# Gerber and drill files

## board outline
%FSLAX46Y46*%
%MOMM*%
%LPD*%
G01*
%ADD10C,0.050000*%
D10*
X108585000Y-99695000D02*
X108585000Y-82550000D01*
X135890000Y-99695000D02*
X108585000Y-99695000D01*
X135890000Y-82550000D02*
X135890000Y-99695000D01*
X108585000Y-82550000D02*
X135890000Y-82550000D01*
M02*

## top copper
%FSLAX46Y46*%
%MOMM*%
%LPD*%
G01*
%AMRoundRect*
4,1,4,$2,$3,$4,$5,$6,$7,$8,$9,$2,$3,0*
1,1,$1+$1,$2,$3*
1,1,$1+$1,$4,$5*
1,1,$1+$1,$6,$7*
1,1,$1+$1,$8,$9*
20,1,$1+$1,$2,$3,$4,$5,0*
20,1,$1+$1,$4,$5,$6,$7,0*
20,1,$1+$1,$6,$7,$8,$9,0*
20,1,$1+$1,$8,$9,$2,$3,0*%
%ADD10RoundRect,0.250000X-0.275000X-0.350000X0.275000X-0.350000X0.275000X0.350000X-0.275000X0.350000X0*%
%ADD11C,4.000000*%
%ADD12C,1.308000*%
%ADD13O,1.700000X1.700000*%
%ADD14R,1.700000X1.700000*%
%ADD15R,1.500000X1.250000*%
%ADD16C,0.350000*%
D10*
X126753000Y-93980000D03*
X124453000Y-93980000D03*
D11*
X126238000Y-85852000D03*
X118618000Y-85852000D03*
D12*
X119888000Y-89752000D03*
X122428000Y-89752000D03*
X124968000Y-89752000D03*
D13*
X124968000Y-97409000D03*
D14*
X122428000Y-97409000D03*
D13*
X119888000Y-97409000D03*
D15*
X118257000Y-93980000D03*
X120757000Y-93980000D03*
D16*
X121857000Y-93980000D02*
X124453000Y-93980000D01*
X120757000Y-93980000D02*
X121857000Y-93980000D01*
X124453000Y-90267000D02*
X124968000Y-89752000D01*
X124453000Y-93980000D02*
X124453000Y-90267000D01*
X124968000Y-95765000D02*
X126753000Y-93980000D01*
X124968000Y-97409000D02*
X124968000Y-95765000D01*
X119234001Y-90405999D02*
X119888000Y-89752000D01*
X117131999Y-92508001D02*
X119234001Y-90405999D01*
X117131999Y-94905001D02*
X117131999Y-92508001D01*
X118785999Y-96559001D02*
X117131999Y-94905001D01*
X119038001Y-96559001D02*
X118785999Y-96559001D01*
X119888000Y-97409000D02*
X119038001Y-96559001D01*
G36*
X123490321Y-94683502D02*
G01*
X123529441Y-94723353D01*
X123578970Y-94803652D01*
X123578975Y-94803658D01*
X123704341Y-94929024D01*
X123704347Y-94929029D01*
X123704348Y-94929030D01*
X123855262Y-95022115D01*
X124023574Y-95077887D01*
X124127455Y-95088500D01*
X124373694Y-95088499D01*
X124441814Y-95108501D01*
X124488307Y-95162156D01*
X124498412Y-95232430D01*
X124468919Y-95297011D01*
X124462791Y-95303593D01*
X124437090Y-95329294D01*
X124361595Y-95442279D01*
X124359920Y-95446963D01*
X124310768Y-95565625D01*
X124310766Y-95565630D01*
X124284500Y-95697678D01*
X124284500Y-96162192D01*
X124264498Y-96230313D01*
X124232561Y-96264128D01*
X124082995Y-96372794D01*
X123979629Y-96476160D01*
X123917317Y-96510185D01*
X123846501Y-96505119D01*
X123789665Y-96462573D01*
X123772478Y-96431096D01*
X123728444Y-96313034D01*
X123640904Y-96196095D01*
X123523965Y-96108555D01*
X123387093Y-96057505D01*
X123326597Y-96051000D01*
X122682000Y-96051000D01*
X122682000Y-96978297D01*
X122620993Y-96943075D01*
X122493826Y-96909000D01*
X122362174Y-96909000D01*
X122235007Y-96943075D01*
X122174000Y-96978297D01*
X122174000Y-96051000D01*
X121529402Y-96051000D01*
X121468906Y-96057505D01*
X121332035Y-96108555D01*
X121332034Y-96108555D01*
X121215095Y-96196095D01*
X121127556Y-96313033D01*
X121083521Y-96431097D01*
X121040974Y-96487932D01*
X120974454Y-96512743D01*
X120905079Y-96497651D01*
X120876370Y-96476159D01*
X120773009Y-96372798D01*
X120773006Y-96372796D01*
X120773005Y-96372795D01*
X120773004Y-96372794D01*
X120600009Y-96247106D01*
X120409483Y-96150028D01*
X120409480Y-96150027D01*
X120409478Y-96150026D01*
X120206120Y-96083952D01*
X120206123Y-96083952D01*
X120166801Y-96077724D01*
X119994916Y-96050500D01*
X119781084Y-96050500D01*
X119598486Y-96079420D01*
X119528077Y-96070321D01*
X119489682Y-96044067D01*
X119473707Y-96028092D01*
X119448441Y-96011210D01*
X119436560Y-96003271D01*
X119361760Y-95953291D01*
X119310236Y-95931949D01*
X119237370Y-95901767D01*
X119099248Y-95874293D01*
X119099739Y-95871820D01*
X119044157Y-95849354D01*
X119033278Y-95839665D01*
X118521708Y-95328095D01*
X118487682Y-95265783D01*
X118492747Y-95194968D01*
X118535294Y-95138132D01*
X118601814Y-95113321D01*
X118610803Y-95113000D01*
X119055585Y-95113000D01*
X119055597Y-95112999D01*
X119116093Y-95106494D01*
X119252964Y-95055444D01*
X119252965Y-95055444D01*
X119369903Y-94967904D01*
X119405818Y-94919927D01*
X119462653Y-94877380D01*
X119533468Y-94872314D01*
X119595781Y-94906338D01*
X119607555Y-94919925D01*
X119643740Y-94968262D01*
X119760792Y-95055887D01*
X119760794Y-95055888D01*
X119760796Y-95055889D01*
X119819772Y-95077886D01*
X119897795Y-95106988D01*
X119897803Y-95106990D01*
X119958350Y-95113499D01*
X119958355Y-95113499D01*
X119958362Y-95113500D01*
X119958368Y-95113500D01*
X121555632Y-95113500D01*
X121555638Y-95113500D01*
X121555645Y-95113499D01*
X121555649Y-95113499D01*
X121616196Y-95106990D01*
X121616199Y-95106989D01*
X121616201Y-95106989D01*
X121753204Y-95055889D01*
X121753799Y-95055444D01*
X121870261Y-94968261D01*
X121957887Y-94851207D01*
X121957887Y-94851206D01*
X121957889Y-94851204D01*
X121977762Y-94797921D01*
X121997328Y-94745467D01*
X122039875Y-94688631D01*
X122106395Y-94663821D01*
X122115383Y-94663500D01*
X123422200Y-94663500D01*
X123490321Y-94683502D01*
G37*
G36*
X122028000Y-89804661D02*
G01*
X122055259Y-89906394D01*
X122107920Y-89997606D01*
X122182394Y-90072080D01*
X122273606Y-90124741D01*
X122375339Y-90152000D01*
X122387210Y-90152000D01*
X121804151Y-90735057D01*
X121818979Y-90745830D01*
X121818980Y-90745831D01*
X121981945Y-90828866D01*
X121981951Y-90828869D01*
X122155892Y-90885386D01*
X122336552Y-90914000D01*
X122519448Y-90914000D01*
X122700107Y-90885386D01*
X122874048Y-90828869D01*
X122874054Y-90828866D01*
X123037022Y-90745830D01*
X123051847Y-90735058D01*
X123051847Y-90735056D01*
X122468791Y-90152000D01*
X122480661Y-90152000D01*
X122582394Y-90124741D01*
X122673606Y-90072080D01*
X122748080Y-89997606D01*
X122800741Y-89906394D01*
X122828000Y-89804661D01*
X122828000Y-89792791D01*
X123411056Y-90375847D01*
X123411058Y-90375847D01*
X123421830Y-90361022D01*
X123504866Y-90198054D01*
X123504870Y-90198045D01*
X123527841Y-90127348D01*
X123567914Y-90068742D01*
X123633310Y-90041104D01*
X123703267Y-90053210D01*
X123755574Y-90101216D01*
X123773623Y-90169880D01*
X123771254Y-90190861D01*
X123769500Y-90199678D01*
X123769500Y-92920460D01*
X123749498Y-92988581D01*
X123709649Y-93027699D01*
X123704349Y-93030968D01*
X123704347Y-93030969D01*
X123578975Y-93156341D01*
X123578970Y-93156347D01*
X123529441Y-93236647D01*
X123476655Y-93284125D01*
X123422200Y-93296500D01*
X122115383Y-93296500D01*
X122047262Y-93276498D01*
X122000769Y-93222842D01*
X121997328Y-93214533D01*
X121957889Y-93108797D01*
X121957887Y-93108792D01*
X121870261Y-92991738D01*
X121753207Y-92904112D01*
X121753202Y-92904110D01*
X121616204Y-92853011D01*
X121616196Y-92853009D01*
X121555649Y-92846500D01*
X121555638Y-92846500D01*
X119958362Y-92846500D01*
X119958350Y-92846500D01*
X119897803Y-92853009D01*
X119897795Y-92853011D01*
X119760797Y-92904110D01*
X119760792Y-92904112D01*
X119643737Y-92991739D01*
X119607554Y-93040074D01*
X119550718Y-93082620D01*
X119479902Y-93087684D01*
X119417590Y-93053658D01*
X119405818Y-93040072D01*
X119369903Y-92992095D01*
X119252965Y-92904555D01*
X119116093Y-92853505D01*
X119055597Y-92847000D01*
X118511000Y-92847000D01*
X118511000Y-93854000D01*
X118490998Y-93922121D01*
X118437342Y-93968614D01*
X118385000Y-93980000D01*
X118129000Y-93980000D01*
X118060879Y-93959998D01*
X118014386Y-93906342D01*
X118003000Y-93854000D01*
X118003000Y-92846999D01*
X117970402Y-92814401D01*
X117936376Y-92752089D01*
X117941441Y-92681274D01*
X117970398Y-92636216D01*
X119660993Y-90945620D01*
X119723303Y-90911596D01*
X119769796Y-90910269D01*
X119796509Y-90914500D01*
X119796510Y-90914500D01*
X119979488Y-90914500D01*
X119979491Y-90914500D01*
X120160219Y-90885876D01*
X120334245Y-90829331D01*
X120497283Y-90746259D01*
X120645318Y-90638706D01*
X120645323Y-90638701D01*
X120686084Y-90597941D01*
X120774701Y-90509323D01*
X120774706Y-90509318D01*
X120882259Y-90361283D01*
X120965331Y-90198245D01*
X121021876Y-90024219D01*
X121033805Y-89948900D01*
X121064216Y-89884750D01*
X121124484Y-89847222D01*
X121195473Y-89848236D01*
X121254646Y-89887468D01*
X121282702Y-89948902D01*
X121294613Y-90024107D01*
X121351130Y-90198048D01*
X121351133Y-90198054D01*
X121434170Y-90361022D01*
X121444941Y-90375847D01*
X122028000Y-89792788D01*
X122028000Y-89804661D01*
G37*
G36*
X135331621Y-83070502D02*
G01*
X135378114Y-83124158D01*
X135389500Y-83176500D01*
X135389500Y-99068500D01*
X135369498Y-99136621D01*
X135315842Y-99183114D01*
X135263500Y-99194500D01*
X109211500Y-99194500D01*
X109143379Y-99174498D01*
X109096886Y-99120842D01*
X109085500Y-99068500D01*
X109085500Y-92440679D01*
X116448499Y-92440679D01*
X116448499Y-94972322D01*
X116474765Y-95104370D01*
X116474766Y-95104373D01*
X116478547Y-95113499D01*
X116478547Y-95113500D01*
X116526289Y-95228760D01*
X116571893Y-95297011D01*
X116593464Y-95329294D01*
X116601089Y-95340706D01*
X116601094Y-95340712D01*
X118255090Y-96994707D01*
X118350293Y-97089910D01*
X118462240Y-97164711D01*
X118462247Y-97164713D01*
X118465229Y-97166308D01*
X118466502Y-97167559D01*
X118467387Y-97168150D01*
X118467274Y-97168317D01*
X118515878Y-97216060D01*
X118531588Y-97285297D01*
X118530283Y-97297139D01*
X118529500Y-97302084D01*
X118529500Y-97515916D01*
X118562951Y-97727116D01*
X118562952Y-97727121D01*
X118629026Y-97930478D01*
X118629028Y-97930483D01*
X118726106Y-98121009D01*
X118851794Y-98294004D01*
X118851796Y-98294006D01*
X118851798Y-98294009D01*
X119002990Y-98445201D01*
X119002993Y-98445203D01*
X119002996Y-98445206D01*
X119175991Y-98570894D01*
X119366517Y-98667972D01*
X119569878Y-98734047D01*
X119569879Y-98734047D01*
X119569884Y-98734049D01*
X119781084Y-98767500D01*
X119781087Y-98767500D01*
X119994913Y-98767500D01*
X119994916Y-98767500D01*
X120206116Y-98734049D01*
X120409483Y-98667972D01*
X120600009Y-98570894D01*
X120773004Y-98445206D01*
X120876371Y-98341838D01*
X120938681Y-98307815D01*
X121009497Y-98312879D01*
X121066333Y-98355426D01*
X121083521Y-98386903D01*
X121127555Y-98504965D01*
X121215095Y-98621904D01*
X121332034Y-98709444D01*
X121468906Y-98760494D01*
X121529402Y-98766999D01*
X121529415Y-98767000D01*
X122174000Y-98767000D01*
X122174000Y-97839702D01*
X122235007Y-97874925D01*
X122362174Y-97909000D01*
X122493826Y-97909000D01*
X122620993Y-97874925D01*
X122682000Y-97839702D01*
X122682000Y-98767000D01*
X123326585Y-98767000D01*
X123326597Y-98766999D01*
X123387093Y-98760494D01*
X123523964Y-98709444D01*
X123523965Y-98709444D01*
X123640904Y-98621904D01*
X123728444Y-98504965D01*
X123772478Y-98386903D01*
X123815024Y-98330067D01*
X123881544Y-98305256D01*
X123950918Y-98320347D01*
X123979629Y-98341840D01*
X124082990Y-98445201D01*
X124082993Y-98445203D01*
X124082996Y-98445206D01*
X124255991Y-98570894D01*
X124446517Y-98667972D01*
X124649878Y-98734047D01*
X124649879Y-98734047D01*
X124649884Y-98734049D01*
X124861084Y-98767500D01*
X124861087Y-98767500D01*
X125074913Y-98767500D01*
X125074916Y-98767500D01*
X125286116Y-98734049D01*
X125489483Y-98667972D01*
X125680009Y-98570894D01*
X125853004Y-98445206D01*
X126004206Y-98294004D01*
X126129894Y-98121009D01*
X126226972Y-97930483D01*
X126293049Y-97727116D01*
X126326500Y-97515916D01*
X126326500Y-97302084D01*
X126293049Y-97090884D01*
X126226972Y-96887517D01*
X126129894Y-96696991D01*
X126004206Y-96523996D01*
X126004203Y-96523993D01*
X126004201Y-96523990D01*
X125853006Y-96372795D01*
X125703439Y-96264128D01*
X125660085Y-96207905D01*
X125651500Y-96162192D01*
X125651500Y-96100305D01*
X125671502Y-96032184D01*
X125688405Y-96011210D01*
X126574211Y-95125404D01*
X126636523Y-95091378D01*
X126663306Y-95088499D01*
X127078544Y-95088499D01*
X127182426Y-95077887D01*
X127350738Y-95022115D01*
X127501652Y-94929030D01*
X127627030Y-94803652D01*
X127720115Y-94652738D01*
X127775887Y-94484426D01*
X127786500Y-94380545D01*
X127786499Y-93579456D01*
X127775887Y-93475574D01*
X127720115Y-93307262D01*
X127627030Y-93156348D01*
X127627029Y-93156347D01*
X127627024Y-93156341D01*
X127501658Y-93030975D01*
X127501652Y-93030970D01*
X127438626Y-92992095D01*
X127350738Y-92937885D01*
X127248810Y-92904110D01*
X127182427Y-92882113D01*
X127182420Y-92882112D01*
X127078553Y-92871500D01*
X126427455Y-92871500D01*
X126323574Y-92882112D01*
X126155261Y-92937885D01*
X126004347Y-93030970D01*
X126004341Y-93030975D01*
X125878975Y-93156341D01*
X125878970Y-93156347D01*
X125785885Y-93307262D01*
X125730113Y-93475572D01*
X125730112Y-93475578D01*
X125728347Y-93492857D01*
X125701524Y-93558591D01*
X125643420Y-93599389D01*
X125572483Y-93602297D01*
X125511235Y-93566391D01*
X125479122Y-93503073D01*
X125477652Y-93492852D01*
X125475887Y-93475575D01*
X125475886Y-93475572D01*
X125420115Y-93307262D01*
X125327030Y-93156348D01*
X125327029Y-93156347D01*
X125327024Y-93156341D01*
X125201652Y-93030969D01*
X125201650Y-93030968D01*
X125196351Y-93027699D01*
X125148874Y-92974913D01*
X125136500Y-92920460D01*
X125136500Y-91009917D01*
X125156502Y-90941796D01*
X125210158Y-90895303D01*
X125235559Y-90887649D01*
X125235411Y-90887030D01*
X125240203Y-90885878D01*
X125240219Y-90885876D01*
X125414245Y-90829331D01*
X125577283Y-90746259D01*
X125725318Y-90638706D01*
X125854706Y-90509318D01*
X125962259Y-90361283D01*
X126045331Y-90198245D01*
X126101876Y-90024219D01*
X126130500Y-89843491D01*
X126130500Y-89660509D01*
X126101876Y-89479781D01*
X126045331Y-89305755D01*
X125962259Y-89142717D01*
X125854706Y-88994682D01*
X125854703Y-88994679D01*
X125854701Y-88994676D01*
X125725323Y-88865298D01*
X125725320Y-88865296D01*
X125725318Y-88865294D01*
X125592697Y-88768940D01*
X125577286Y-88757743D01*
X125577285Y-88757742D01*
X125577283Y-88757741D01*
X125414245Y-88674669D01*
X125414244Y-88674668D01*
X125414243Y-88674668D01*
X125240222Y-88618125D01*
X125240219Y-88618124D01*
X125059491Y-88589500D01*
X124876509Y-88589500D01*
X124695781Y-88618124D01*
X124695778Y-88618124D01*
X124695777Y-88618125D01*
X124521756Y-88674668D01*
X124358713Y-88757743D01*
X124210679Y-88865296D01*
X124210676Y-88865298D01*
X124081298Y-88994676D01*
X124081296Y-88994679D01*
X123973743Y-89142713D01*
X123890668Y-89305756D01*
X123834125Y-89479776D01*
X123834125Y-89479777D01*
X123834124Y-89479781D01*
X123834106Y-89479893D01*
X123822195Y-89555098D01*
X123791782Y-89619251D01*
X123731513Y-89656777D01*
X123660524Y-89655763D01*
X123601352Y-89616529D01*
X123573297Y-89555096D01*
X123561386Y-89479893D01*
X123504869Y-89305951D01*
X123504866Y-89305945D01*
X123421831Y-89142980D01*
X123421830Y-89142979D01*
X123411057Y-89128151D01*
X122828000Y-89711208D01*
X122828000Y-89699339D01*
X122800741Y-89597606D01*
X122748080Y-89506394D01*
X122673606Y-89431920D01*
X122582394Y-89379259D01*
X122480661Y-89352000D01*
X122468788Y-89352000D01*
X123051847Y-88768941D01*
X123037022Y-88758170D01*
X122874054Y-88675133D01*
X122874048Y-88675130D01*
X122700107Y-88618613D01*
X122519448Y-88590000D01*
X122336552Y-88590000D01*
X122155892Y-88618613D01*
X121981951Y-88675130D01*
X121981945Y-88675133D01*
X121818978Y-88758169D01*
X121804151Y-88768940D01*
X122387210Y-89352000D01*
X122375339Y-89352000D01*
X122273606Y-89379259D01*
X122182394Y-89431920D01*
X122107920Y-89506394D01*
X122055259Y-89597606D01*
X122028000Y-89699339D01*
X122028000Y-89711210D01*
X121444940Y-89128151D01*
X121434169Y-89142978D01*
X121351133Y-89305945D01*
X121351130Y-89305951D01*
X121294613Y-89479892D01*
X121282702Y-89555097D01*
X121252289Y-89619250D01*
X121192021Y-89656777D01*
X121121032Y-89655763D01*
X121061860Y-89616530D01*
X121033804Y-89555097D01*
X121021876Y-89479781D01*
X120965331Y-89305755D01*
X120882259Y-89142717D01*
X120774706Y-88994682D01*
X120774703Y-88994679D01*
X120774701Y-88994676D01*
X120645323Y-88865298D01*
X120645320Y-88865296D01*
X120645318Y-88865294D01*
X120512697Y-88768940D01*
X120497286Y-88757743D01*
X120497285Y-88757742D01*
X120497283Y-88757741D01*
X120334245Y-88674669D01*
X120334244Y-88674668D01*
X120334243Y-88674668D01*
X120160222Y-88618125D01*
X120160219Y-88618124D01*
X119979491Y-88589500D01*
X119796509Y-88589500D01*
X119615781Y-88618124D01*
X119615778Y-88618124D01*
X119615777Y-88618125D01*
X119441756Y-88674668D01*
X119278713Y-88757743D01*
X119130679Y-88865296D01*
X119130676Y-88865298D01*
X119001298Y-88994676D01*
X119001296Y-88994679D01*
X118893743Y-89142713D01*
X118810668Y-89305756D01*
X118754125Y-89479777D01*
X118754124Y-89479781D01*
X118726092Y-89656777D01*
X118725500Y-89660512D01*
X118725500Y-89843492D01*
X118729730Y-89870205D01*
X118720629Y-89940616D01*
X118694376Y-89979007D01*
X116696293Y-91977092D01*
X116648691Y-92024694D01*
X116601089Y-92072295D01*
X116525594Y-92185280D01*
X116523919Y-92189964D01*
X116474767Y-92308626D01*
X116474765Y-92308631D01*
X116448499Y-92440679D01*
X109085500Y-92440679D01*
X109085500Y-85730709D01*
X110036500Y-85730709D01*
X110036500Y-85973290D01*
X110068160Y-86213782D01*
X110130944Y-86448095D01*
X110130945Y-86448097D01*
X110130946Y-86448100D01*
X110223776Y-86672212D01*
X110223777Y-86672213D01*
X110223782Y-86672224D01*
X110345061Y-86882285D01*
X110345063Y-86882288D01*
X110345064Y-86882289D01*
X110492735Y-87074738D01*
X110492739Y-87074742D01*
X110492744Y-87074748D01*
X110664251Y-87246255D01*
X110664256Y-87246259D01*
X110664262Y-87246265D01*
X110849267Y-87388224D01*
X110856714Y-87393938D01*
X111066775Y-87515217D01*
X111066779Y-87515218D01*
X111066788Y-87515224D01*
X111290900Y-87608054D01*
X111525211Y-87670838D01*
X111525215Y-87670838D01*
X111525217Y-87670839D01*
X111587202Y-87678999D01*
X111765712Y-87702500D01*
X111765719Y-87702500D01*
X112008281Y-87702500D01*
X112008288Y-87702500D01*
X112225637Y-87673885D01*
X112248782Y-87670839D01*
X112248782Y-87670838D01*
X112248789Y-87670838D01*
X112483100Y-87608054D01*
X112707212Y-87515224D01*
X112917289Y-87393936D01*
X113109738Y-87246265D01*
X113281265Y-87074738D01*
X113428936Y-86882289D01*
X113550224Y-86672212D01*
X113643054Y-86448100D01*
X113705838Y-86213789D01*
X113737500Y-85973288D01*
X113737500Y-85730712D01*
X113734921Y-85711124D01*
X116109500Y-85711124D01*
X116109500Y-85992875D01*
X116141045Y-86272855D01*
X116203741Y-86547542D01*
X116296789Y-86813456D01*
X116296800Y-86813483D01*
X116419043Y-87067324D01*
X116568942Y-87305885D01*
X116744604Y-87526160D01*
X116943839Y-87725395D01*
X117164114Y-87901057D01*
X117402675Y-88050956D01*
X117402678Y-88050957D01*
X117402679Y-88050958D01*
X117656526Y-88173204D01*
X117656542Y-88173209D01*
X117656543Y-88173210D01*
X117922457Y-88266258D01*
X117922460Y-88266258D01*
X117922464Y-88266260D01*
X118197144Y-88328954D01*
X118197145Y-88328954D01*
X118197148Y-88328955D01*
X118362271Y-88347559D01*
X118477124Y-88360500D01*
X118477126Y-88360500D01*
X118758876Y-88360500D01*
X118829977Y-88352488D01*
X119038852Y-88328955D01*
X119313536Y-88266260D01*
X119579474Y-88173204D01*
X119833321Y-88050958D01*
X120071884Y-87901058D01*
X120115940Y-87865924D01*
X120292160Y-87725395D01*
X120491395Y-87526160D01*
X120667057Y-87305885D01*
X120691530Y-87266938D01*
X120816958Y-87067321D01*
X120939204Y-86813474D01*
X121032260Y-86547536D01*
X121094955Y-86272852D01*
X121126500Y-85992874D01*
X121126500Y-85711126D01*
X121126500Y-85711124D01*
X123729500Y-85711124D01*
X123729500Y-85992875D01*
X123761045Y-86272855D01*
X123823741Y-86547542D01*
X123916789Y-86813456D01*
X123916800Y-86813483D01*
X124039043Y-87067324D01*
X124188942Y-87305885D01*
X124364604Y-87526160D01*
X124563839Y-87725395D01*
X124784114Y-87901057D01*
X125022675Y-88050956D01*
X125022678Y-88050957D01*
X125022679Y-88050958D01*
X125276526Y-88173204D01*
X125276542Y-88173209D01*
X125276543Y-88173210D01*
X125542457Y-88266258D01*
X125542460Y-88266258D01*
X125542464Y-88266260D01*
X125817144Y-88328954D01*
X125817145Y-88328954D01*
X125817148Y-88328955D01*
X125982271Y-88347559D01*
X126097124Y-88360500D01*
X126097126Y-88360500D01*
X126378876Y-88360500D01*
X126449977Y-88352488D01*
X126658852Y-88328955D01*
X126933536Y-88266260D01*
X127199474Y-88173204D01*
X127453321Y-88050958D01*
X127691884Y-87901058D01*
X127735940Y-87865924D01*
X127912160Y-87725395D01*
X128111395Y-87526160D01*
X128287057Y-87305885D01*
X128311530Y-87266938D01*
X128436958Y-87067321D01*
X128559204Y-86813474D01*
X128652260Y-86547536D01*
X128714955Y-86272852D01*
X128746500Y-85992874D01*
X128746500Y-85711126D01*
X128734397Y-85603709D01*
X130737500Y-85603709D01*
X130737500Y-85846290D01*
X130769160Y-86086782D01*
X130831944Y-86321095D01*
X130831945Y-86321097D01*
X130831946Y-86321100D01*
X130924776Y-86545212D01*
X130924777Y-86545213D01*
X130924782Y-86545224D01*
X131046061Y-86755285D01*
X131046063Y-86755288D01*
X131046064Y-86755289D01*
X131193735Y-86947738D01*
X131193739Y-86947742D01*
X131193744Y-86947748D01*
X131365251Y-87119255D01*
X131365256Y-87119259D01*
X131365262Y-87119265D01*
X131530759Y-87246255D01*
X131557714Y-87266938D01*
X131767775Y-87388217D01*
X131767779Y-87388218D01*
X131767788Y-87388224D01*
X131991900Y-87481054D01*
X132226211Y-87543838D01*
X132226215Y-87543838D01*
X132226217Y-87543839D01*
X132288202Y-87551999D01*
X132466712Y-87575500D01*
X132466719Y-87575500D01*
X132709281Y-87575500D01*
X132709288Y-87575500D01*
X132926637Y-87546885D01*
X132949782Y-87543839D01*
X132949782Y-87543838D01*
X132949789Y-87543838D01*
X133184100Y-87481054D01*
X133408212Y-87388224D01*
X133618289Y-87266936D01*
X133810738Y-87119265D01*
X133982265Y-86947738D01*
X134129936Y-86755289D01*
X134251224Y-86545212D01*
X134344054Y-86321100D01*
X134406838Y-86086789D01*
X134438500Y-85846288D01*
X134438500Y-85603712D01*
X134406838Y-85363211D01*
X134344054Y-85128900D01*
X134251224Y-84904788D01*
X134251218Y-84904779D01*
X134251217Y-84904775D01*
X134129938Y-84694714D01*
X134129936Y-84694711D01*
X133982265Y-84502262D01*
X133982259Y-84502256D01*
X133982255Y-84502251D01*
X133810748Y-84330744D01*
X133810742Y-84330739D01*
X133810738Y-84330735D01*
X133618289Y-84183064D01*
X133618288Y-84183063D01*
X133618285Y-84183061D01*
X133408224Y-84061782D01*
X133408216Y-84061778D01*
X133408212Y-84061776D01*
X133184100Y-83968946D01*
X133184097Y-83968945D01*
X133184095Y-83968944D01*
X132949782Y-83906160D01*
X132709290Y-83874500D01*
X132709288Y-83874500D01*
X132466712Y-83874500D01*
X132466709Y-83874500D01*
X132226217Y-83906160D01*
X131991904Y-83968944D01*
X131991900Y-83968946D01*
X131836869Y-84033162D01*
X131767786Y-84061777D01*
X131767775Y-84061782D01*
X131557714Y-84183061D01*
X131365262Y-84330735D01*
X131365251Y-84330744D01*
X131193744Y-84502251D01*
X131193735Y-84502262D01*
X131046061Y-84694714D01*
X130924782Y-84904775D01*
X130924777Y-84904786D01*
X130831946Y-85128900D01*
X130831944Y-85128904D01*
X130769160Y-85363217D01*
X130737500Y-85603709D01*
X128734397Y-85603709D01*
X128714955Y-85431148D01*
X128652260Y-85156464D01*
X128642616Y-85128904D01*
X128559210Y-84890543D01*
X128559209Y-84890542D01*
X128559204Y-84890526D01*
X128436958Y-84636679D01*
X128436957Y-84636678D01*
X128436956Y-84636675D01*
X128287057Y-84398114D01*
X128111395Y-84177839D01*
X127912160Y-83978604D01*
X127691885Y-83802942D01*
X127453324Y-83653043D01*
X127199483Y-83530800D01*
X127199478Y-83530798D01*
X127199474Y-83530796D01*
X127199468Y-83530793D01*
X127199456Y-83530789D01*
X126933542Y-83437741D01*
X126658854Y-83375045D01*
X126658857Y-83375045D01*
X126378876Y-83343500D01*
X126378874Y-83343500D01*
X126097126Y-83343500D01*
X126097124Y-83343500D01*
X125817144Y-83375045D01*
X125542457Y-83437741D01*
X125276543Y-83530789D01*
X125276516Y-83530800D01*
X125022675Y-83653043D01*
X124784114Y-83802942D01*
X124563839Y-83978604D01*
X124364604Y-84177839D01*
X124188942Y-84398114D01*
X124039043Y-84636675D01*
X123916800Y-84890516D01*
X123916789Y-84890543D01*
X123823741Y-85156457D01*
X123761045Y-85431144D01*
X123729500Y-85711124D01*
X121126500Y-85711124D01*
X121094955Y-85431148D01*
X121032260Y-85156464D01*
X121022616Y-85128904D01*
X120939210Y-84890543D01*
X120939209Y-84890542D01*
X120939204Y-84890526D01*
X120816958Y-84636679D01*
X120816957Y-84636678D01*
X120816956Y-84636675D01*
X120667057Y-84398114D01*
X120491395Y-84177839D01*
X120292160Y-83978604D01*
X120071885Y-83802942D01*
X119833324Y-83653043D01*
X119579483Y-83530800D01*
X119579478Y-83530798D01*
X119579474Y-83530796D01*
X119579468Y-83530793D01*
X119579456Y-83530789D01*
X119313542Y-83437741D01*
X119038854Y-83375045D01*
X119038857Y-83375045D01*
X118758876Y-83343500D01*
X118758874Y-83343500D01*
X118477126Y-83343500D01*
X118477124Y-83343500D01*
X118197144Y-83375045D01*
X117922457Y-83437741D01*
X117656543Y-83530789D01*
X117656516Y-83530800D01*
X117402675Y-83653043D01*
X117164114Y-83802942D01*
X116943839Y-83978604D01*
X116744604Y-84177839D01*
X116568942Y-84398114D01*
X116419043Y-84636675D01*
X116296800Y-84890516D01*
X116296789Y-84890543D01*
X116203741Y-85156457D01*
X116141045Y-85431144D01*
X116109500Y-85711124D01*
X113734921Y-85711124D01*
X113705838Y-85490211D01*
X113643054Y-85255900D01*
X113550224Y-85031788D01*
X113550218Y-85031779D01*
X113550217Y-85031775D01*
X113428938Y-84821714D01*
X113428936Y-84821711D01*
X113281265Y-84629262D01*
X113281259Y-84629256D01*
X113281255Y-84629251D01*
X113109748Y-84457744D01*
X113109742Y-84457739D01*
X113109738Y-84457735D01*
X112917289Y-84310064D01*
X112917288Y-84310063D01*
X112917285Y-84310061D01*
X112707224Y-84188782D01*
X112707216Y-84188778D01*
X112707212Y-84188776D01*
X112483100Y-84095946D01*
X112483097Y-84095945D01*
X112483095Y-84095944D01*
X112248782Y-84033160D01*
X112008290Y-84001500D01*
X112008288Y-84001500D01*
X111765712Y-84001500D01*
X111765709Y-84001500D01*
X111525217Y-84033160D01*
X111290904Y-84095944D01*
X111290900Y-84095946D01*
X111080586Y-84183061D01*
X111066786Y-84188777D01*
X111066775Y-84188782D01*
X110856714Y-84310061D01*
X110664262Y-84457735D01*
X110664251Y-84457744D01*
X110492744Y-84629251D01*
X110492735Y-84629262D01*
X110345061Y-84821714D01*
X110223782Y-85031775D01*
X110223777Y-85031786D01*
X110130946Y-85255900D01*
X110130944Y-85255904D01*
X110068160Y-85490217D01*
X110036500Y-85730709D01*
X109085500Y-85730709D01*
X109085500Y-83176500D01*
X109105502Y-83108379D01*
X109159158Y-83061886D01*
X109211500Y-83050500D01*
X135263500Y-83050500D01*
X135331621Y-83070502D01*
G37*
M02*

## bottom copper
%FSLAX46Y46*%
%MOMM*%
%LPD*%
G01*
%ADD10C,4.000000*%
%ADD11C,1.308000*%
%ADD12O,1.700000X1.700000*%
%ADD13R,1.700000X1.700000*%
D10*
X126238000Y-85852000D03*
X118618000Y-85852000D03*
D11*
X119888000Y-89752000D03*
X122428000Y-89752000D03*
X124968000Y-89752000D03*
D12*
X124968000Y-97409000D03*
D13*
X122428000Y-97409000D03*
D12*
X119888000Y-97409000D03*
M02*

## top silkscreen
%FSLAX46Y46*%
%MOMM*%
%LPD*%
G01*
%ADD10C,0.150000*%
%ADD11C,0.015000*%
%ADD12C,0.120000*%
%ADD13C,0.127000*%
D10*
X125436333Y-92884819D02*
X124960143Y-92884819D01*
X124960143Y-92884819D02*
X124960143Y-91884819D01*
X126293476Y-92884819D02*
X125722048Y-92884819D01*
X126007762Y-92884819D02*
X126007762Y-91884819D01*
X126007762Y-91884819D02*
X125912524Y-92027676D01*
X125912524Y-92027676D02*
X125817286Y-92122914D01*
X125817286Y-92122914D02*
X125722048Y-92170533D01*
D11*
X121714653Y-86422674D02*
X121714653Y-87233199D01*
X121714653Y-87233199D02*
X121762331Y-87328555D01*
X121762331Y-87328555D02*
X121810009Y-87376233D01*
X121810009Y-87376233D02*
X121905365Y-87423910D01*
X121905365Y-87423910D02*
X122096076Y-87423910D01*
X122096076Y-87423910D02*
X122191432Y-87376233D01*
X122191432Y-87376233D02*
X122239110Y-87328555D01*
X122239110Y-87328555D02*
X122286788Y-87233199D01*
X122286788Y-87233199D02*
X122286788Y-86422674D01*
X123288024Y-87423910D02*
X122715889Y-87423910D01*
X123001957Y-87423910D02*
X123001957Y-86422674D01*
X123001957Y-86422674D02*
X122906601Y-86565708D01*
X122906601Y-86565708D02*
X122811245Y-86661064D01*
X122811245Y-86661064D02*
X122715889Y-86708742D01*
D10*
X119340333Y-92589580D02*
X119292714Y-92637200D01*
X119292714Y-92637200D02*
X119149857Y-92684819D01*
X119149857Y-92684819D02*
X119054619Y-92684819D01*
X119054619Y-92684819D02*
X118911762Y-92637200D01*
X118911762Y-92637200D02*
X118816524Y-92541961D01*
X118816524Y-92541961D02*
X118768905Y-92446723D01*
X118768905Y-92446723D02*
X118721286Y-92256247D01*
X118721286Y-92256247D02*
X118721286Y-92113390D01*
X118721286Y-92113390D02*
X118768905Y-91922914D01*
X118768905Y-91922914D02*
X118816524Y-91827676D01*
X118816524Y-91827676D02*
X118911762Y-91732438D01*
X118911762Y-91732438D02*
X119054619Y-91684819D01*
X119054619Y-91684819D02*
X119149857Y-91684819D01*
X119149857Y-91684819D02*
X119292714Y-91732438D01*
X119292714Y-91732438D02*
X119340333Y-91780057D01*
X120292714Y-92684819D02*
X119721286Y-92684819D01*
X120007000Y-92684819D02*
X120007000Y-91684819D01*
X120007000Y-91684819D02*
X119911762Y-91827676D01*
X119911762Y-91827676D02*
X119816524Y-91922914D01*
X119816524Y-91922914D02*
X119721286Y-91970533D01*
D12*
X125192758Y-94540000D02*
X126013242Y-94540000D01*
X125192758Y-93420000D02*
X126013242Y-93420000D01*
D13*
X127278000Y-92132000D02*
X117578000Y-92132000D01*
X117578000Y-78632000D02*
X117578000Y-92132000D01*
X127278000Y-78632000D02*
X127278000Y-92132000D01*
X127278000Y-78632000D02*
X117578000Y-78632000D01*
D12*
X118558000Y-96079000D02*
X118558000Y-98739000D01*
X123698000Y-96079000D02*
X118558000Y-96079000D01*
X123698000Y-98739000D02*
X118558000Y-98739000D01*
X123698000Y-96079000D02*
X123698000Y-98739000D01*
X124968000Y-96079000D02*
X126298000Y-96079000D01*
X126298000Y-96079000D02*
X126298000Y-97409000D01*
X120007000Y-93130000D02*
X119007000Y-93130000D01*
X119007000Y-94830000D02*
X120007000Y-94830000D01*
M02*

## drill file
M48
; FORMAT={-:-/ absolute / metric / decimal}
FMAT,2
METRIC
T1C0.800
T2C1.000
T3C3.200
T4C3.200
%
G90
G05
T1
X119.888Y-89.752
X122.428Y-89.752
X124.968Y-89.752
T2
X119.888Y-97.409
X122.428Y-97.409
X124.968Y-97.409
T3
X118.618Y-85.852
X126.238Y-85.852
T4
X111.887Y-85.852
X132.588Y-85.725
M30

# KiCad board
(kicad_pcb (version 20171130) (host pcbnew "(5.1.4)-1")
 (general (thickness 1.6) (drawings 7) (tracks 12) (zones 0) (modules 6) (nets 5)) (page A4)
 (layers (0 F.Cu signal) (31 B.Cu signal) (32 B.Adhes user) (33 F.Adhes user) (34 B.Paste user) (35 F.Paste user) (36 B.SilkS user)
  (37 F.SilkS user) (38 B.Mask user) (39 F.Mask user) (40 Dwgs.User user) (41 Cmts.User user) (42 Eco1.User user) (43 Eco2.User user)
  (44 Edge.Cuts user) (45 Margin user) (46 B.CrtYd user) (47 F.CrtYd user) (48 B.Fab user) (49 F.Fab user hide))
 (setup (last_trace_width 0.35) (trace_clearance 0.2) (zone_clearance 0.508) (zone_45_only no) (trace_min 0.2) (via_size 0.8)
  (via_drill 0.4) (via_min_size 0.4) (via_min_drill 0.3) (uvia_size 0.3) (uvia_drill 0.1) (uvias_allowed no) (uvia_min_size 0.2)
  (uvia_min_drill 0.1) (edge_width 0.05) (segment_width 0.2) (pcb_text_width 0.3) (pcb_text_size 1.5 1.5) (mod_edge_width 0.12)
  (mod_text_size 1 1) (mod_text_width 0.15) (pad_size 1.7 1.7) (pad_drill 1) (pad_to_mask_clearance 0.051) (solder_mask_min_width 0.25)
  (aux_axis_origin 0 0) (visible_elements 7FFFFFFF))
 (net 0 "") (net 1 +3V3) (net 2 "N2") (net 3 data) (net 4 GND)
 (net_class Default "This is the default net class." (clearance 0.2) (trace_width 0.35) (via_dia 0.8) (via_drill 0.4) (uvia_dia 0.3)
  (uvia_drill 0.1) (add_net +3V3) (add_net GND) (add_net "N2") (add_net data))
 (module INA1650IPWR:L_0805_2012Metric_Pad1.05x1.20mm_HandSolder (layer F.Cu) (at 125.603 93.98)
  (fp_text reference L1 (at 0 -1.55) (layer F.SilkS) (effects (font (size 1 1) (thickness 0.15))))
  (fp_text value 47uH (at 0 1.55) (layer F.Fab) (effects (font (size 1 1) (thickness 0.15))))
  (fp_line (start -0.410242 0.56) (end 0.410242 0.56) (layer F.SilkS) (width 0.12))
  (fp_line (start -0.410242 -0.56) (end 0.410242 -0.56) (layer F.SilkS) (width 0.12))
  (pad 2 smd roundrect (at 1.15 0) (size 1.05 1.2) (layers F.Cu F.Paste F.Mask) (roundrect_rratio 0.238095) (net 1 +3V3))
  (pad 1 smd roundrect (at -1.15 0) (size 1.05 1.2) (layers F.Cu F.Paste F.Mask) (roundrect_rratio 0.238095) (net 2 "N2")))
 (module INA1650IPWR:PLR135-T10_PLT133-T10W (layer F.Cu) (at 122.428 87.122)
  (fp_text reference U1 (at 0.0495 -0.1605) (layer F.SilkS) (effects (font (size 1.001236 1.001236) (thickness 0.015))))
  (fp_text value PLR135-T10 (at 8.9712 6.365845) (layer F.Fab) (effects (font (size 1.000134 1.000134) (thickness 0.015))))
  (fp_line (start 4.85 5.01) (end -4.85 5.01) (layer F.SilkS) (width 0.127))
  (fp_line (start -4.85 -8.49) (end -4.85 5.01) (layer F.SilkS) (width 0.127))
  (fp_line (start 4.85 -8.49) (end 4.85 5.01) (layer F.SilkS) (width 0.127))
  (fp_line (start 4.85 -8.49) (end -4.85 -8.49) (layer F.SilkS) (width 0.127))
  (pad NC1 thru_hole circle (at 3.81 -1.27) (size 4 4) (drill 3.2) (layers *.Cu *.Mask))
  (pad NC2 thru_hole circle (at -3.81 -1.27) (size 4 4) (drill 3.2) (layers *.Cu *.Mask))
  (pad 3 thru_hole circle (at -2.54 2.63) (size 1.308 1.308) (drill 0.8) (layers *.Cu *.Mask) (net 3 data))
  (pad 2 thru_hole circle (at 0 2.63) (size 1.308 1.308) (drill 0.8) (layers *.Cu *.Mask) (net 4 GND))
  (pad 1 thru_hole circle (at 2.54 2.63) (size 1.308 1.308) (drill 0.8) (layers *.Cu *.Mask) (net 2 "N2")))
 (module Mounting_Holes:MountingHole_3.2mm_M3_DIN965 (layer F.Cu) (at 132.588 85.725)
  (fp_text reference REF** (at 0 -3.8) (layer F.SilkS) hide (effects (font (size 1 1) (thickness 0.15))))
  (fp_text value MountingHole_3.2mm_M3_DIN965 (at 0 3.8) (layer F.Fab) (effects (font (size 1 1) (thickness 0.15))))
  (pad 1 np_thru_hole circle (at 0 0) (size 3.2 3.2) (drill 3.2) (layers *.Cu *.Mask)))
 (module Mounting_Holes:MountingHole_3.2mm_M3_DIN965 (layer F.Cu) (at 111.887 85.852)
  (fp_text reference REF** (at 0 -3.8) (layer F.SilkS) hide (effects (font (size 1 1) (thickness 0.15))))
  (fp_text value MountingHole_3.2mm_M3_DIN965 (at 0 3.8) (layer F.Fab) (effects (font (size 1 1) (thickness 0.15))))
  (pad 1 np_thru_hole circle (at 0 0) (size 3.2 3.2) (drill 3.2) (layers *.Cu *.Mask)))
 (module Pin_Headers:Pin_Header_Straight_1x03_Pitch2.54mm (layer F.Cu) (at 124.968 97.409 270)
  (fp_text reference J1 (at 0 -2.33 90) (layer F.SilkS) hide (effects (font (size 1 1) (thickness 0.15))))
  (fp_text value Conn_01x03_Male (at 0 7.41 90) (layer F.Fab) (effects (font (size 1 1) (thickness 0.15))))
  (fp_line (start -1.33 6.41) (end 1.33 6.41) (layer F.SilkS) (width 0.12))
  (fp_line (start -1.33 1.27) (end -1.33 6.41) (layer F.SilkS) (width 0.12))
  (fp_line (start 1.33 1.27) (end 1.33 6.41) (layer F.SilkS) (width 0.12))
  (fp_line (start -1.33 1.27) (end 1.33 1.27) (layer F.SilkS) (width 0.12))
  (fp_line (start -1.33 0) (end -1.33 -1.33) (layer F.SilkS) (width 0.12))
  (fp_line (start -1.33 -1.33) (end 0 -1.33) (layer F.SilkS) (width 0.12))
  (pad 1 thru_hole oval (at 0 0 270) (size 1.7 1.7) (drill 1) (layers *.Cu *.Mask) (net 1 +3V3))
  (pad 2 thru_hole rect (at 0 2.54 270) (size 1.7 1.7) (drill 1) (layers *.Cu *.Mask) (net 4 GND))
  (pad 3 thru_hole oval (at 0 5.08 270) (size 1.7 1.7) (drill 1) (layers *.Cu *.Mask) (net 3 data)))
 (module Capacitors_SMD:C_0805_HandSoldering (layer F.Cu) (at 119.507 93.98)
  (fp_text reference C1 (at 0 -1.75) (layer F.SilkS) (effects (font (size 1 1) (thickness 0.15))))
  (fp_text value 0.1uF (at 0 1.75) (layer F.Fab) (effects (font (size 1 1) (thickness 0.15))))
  (fp_line (start 0.5 -0.85) (end -0.5 -0.85) (layer F.SilkS) (width 0.12))
  (fp_line (start -0.5 0.85) (end 0.5 0.85) (layer F.SilkS) (width 0.12))
  (pad 1 smd rect (at -1.25 0) (size 1.5 1.25) (layers F.Cu F.Paste F.Mask) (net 4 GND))
  (pad 2 smd rect (at 1.25 0) (size 1.5 1.25) (layers F.Cu F.Paste F.Mask) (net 2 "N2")))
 (gr_line (start 108.585 99.695) (end 108.585 82.55) (layer Edge.Cuts) (width 0.05))
 (gr_line (start 135.89 99.695) (end 108.585 99.695) (layer Edge.Cuts) (width 0.05))
 (gr_line (start 135.89 82.55) (end 135.89 99.695) (layer Edge.Cuts) (width 0.05))
 (gr_line (start 108.585 82.55) (end 135.89 82.55) (layer Edge.Cuts) (width 0.05))
 (segment (start 121.857 93.98) (end 124.453 93.98) (width 0.35) (layer F.Cu) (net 2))
 (segment (start 120.757 93.98) (end 121.857 93.98) (width 0.35) (layer F.Cu) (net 2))
 (segment (start 124.453 90.267) (end 124.968 89.752) (width 0.35) (layer F.Cu) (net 2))
 (segment (start 124.453 93.98) (end 124.453 90.267) (width 0.35) (layer F.Cu) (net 2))
 (segment (start 124.968 95.765) (end 126.753 93.98) (width 0.35) (layer F.Cu) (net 1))
 (segment (start 124.968 97.409) (end 124.968 95.765) (width 0.35) (layer F.Cu) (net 1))
 (segment (start 119.234001 90.405999) (end 119.888 89.752) (width 0.35) (layer F.Cu) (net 3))
 (segment (start 117.131999 92.508001) (end 119.234001 90.405999) (width 0.35) (layer F.Cu) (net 3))
 (segment (start 117.131999 94.905001) (end 117.131999 92.508001) (width 0.35) (layer F.Cu) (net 3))
 (segment (start 118.785999 96.559001) (end 117.131999 94.905001) (width 0.35) (layer F.Cu) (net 3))
 (segment (start 119.038001 96.559001) (end 118.785999 96.559001) (width 0.35) (layer F.Cu) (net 3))
 (segment (start 119.888 97.409) (end 119.038001 96.559001) (width 0.35) (layer F.Cu) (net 3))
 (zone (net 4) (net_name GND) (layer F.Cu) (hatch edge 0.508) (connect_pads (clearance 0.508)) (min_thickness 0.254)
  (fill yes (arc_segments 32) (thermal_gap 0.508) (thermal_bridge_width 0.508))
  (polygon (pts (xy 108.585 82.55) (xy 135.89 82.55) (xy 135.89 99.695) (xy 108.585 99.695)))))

